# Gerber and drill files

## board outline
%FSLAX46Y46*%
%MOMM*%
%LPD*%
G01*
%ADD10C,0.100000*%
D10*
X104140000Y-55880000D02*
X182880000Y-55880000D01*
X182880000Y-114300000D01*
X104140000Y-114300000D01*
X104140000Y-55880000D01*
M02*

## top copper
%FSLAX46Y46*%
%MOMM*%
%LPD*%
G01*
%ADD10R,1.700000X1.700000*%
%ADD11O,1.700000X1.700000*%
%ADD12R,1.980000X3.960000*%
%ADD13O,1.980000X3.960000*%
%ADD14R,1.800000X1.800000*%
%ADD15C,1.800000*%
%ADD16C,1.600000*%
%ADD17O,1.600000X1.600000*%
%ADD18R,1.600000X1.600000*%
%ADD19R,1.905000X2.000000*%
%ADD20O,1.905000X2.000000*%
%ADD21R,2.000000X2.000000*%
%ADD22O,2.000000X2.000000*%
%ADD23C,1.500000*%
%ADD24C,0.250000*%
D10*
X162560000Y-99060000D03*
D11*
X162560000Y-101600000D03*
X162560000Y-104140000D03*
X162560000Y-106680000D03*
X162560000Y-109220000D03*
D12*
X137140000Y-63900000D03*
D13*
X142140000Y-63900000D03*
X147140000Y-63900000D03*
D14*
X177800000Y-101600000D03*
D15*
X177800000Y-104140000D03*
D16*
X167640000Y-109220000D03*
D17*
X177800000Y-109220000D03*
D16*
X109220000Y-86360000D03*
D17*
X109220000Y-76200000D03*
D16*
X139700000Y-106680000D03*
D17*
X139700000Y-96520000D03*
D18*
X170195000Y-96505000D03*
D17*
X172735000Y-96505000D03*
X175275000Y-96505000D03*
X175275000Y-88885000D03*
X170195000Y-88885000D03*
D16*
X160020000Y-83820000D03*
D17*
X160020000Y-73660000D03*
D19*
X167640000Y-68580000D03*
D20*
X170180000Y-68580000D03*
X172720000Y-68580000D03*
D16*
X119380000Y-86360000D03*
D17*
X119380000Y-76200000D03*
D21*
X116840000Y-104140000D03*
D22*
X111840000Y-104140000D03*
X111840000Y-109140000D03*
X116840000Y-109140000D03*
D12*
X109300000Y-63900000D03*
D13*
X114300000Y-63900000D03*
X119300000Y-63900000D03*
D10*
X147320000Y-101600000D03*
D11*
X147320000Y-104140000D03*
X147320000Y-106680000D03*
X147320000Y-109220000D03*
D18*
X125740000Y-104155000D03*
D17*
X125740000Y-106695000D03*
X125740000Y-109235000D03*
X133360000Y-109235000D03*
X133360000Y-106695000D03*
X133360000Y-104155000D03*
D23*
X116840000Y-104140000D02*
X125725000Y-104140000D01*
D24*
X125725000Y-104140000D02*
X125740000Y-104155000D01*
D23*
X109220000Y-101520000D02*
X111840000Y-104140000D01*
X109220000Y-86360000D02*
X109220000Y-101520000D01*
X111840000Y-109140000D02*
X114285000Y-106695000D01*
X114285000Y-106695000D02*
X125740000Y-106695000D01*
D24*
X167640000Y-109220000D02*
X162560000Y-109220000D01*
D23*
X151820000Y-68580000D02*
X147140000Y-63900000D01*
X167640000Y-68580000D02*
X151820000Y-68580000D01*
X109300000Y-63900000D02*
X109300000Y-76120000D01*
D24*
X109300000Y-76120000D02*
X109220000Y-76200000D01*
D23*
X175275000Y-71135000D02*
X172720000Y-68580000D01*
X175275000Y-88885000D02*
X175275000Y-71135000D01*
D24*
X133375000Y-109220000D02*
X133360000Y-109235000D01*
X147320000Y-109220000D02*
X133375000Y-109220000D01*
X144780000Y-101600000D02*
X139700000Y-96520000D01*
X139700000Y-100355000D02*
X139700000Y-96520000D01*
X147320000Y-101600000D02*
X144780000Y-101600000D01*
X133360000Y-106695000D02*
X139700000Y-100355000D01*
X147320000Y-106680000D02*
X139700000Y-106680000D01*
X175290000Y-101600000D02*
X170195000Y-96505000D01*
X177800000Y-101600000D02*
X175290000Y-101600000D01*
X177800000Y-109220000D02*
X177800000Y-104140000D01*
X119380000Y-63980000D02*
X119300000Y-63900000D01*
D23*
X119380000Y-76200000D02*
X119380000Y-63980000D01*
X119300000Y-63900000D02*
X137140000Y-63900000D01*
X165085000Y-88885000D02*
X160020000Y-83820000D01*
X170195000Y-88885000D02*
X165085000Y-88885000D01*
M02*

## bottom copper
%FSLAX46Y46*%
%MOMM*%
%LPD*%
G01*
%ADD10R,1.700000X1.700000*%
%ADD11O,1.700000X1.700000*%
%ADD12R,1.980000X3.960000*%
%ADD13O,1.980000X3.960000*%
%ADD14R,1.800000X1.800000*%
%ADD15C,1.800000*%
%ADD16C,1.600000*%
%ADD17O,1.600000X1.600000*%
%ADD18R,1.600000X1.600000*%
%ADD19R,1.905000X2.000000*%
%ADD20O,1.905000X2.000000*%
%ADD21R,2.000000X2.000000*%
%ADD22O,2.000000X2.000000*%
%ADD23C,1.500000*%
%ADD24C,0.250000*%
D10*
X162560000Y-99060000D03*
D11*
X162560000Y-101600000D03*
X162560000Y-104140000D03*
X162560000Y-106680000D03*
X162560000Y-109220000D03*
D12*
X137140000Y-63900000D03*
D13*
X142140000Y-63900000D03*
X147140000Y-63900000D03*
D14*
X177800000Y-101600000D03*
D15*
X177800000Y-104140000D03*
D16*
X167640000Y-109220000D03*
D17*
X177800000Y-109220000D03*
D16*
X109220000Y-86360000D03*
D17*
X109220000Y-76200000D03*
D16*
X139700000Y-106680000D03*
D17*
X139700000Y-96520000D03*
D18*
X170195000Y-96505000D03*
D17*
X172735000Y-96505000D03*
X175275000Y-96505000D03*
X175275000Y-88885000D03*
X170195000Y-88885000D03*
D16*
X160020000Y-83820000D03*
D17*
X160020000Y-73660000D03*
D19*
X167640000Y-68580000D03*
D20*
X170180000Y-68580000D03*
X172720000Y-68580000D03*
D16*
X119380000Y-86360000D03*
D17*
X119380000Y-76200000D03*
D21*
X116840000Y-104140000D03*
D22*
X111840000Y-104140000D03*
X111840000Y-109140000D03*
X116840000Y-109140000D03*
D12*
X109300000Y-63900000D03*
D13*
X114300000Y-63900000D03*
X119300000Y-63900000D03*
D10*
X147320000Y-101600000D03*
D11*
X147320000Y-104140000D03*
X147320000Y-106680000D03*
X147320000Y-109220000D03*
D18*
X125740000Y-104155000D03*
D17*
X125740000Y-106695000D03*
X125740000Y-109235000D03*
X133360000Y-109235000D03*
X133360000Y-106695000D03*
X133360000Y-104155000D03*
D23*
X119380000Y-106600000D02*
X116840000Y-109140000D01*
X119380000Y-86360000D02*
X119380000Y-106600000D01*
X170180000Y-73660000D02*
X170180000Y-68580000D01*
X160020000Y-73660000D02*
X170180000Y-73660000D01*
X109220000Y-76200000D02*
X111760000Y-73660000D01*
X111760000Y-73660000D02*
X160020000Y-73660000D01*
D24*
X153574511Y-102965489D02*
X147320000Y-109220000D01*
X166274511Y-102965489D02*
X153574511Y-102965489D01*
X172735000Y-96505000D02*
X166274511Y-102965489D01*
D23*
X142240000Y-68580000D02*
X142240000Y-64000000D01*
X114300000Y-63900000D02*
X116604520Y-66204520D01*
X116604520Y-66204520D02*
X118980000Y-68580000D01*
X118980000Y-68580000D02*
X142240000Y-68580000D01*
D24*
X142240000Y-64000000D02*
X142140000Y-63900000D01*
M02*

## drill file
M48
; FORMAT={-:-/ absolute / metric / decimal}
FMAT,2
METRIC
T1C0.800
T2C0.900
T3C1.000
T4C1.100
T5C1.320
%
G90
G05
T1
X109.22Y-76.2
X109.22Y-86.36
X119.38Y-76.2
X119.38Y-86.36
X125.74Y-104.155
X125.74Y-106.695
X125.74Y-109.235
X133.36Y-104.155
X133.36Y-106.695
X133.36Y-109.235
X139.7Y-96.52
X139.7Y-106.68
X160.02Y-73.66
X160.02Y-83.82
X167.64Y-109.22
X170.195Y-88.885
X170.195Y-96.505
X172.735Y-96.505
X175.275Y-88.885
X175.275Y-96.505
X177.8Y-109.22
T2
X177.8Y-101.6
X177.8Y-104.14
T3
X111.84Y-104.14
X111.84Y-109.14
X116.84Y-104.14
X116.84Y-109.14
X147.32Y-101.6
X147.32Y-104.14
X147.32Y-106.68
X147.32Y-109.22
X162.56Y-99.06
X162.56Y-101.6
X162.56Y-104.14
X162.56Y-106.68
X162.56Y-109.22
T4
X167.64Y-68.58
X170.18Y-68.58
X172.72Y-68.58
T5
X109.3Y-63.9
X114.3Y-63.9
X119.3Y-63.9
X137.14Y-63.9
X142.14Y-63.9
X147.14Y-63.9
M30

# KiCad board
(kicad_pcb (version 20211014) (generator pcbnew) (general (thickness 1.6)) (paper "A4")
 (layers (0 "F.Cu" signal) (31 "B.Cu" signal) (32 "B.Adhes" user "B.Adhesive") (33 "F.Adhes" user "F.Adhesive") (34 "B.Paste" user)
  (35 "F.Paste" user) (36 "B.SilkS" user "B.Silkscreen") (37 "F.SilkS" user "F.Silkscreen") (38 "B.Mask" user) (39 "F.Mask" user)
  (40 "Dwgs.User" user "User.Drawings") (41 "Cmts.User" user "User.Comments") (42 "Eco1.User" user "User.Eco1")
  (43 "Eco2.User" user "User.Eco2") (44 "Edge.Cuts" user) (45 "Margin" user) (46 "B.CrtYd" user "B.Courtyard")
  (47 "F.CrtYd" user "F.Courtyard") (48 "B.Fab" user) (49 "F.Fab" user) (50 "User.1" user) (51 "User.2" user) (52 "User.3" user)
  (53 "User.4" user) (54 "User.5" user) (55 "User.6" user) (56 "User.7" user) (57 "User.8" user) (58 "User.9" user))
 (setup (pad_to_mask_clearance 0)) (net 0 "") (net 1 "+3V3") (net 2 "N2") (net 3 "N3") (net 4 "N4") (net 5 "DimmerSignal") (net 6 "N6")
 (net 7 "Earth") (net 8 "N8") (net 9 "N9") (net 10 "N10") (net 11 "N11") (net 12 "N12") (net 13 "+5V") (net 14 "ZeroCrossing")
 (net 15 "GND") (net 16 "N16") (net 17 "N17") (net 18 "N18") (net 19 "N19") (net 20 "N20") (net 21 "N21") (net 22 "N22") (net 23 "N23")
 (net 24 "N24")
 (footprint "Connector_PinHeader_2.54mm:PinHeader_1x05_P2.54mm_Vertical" (layer "F.Cu") (at 162.56 99.06)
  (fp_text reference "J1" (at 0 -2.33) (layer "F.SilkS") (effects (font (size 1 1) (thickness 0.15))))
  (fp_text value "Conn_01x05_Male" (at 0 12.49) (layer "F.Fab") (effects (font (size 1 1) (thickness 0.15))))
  (pad "1" thru_hole rect (at 0 0) (size 1.7 1.7) (drill 1) (layers *.Cu *.Mask) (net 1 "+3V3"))
  (pad "2" thru_hole oval (at 0 2.54) (size 1.7 1.7) (drill 1) (layers *.Cu *.Mask) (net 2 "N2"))
  (pad "3" thru_hole oval (at 0 5.08) (size 1.7 1.7) (drill 1) (layers *.Cu *.Mask) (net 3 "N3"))
  (pad "4" thru_hole oval (at 0 7.62) (size 1.7 1.7) (drill 1) (layers *.Cu *.Mask) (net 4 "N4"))
  (pad "5" thru_hole oval (at 0 10.16) (size 1.7 1.7) (drill 1) (layers *.Cu *.Mask) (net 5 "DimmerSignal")))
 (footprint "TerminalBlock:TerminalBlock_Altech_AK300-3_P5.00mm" (layer "F.Cu") (at 137.14 63.9)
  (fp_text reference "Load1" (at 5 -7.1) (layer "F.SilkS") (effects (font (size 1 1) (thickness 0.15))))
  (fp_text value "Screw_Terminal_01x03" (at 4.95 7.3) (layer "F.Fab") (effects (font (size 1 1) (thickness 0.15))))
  (pad "1" thru_hole rect (at 0 0) (size 1.98 3.96) (drill 1.32) (layers *.Cu *.Mask) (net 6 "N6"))
  (pad "2" thru_hole oval (at 5 0) (size 1.98 3.96) (drill 1.32) (layers *.Cu *.Mask) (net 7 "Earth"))
  (pad "3" thru_hole oval (at 10 0) (size 1.98 3.96) (drill 1.32) (layers *.Cu *.Mask) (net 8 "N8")))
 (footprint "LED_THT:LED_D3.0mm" (layer "F.Cu") (at 177.8 101.6 -90)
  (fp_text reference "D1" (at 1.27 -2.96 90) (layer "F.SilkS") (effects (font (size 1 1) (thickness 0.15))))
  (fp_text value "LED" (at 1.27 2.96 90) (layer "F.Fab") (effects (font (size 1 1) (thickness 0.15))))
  (pad "1" thru_hole rect (at 0 0 270) (size 1.8 1.8) (drill 0.9) (layers *.Cu *.Mask) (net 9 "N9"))
  (pad "2" thru_hole circle (at 2.54 0 270) (size 1.8 1.8) (drill 0.9) (layers *.Cu *.Mask) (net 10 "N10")))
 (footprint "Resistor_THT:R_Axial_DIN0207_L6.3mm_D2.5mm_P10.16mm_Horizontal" (layer "F.Cu") (at 167.64 109.22)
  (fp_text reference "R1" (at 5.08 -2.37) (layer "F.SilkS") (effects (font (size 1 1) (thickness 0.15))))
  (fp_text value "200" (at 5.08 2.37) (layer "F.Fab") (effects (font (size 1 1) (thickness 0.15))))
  (pad "1" thru_hole circle (at 0 0) (size 1.6 1.6) (drill 0.8) (layers *.Cu *.Mask) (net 5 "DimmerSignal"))
  (pad "2" thru_hole oval (at 10.16 0) (size 1.6 1.6) (drill 0.8) (layers *.Cu *.Mask) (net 10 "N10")))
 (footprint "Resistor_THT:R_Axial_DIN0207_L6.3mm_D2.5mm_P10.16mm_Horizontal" (layer "F.Cu") (at 109.22 86.36 90)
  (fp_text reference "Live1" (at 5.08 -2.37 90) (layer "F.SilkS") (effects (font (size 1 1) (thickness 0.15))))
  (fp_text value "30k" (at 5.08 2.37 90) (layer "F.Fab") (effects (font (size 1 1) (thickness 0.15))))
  (pad "1" thru_hole circle (at 0 0 90) (size 1.6 1.6) (drill 0.8) (layers *.Cu *.Mask) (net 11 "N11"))
  (pad "2" thru_hole oval (at 10.16 0 90) (size 1.6 1.6) (drill 0.8) (layers *.Cu *.Mask) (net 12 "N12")))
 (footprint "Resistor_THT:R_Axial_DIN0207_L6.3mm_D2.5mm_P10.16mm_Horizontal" (layer "F.Cu") (at 139.7 106.68 90)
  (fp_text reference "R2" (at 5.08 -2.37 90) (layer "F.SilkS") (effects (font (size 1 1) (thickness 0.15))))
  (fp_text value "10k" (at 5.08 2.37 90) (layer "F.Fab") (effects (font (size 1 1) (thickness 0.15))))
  (pad "1" thru_hole circle (at 0 0 90) (size 1.6 1.6) (drill 0.8) (layers *.Cu *.Mask) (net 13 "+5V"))
  (pad "2" thru_hole oval (at 10.16 0 90) (size 1.6 1.6) (drill 0.8) (layers *.Cu *.Mask) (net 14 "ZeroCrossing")))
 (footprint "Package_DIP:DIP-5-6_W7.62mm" (layer "F.Cu") (at 170.195 96.505 90)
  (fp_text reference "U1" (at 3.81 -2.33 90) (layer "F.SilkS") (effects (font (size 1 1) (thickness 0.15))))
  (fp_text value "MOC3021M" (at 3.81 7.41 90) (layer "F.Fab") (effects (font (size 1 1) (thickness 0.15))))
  (pad "1" thru_hole rect (at 0 0 90) (size 1.6 1.6) (drill 0.8) (layers *.Cu *.Mask) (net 9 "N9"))
  (pad "2" thru_hole oval (at 0 2.54 90) (size 1.6 1.6) (drill 0.8) (layers *.Cu *.Mask) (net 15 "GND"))
  (pad "3" thru_hole oval (at 0 5.08 90) (size 1.6 1.6) (drill 0.8) (layers *.Cu *.Mask) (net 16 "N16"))
  (pad "4" thru_hole oval (at 7.62 5.08 90) (size 1.6 1.6) (drill 0.8) (layers *.Cu *.Mask) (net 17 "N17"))
  (pad "6" thru_hole oval (at 7.62 0 90) (size 1.6 1.6) (drill 0.8) (layers *.Cu *.Mask) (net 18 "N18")))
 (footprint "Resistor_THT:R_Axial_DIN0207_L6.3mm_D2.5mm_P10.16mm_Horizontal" (layer "F.Cu") (at 160.02 83.82 90)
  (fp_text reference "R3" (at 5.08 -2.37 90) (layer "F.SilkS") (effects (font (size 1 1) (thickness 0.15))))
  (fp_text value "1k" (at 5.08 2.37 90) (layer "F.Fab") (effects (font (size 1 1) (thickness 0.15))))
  (pad "1" thru_hole circle (at 0 0 90) (size 1.6 1.6) (drill 0.8) (layers *.Cu *.Mask) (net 18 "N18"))
  (pad "2" thru_hole oval (at 10.16 0 90) (size 1.6 1.6) (drill 0.8) (layers *.Cu *.Mask) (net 12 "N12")))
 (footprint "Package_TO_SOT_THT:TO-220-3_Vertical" (layer "F.Cu") (at 167.64 68.58)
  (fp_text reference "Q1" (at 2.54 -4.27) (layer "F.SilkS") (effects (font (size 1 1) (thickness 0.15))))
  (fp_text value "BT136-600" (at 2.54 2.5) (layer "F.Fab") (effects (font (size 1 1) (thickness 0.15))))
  (pad "1" thru_hole rect (at 0 0) (size 1.905 2) (drill 1.1) (layers *.Cu *.Mask) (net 8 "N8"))
  (pad "2" thru_hole oval (at 2.54 0) (size 1.905 2) (drill 1.1) (layers *.Cu *.Mask) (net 12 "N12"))
  (pad "3" thru_hole oval (at 5.08 0) (size 1.905 2) (drill 1.1) (layers *.Cu *.Mask) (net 17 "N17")))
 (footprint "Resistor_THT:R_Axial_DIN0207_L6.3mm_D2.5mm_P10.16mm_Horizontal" (layer "F.Cu") (at 119.38 86.36 90)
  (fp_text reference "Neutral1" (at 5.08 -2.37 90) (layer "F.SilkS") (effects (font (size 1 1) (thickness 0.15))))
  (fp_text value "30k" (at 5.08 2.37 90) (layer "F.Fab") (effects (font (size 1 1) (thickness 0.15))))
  (pad "1" thru_hole circle (at 0 0 90) (size 1.6 1.6) (drill 0.8) (layers *.Cu *.Mask) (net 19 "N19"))
  (pad "2" thru_hole oval (at 10.16 0 90) (size 1.6 1.6) (drill 0.8) (layers *.Cu *.Mask) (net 6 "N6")))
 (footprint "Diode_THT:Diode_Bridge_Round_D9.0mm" (layer "F.Cu") (at 116.84 104.14 -90)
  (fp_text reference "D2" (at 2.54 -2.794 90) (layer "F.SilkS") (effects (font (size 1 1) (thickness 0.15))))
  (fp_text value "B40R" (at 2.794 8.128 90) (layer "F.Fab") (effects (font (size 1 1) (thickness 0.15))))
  (pad "1" thru_hole rect (at 0 0 270) (size 2 2) (drill 1) (layers *.Cu *.Mask) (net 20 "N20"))
  (pad "2" thru_hole oval (at 0 5 270) (size 2 2) (drill 1) (layers *.Cu *.Mask) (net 11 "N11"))
  (pad "3" thru_hole oval (at 5 5 270) (size 2 2) (drill 1) (layers *.Cu *.Mask) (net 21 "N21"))
  (pad "4" thru_hole oval (at 5 0 270) (size 2 2) (drill 1) (layers *.Cu *.Mask) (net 19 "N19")))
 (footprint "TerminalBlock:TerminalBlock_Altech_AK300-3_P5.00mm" (layer "F.Cu") (at 109.3 63.9)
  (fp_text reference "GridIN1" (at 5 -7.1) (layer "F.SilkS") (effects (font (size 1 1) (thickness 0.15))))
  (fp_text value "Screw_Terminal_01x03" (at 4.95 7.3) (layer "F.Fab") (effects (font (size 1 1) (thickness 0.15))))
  (pad "1" thru_hole rect (at 0 0) (size 1.98 3.96) (drill 1.32) (layers *.Cu *.Mask) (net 12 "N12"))
  (pad "2" thru_hole oval (at 5 0) (size 1.98 3.96) (drill 1.32) (layers *.Cu *.Mask) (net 7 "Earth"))
  (pad "3" thru_hole oval (at 10 0) (size 1.98 3.96) (drill 1.32) (layers *.Cu *.Mask) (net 6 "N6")))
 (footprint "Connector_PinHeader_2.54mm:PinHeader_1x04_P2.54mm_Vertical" (layer "F.Cu") (at 147.32 101.6)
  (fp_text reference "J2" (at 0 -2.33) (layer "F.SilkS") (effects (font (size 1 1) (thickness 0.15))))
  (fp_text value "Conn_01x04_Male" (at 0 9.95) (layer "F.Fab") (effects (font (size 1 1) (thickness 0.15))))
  (pad "1" thru_hole rect (at 0 0) (size 1.7 1.7) (drill 1) (layers *.Cu *.Mask) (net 14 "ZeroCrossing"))
  (pad "2" thru_hole oval (at 0 2.54) (size 1.7 1.7) (drill 1) (layers *.Cu *.Mask) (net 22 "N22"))
  (pad "3" thru_hole oval (at 0 5.08) (size 1.7 1.7) (drill 1) (layers *.Cu *.Mask) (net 13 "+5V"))
  (pad "4" thru_hole oval (at 0 7.62) (size 1.7 1.7) (drill 1) (layers *.Cu *.Mask) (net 15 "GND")))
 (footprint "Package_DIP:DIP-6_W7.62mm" (layer "F.Cu") (at 125.74 104.155)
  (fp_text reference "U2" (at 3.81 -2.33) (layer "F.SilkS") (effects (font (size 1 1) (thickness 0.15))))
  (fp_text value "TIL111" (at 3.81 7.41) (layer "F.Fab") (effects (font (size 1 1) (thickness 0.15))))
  (pad "1" thru_hole rect (at 0 0) (size 1.6 1.6) (drill 0.8) (layers *.Cu *.Mask) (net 20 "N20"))
  (pad "2" thru_hole oval (at 0 2.54) (size 1.6 1.6) (drill 0.8) (layers *.Cu *.Mask) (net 21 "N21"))
  (pad "3" thru_hole oval (at 0 5.08) (size 1.6 1.6) (drill 0.8) (layers *.Cu *.Mask) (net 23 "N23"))
  (pad "4" thru_hole oval (at 7.62 5.08) (size 1.6 1.6) (drill 0.8) (layers *.Cu *.Mask) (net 15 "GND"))
  (pad "5" thru_hole oval (at 7.62 2.54) (size 1.6 1.6) (drill 0.8) (layers *.Cu *.Mask) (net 14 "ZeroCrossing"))
  (pad "6" thru_hole oval (at 7.62 0) (size 1.6 1.6) (drill 0.8) (layers *.Cu *.Mask) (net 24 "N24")))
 (gr_rect (start 104.14 55.88) (end 182.88 114.3) (layer "Edge.Cuts") (width 0.1) (fill none))
 (segment (start 116.84 104.14) (end 125.725 104.14) (width 1.5) (layer "F.Cu") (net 20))
 (segment (start 125.725 104.14) (end 125.74 104.155) (width 0.25) (layer "F.Cu") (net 20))
 (segment (start 109.22 101.52) (end 111.84 104.14) (width 1.5) (layer "F.Cu") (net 11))
 (segment (start 109.22 86.36) (end 109.22 101.52) (width 1.5) (layer "F.Cu") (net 11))
 (segment (start 111.84 109.14) (end 114.285 106.695) (width 1.5) (layer "F.Cu") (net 21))
 (segment (start 114.285 106.695) (end 125.74 106.695) (width 1.5) (layer "F.Cu") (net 21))
 (segment (start 119.38 106.6) (end 116.84 109.14) (width 1.5) (layer "B.Cu") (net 19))
 (segment (start 119.38 86.36) (end 119.38 106.6) (width 1.5) (layer "B.Cu") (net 19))
 (segment (start 167.64 109.22) (end 162.56 109.22) (width 0.25) (layer "F.Cu") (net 5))
 (segment (start 151.82 68.58) (end 147.14 63.9) (width 1.5) (layer "F.Cu") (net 8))
 (segment (start 167.64 68.58) (end 151.82 68.58) (width 1.5) (layer "F.Cu") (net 8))
 (segment (start 109.3 63.9) (end 109.3 76.12) (width 1.5) (layer "F.Cu") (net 12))
 (segment (start 109.3 76.12) (end 109.22 76.2) (width 0.25) (layer "F.Cu") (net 12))
 (segment (start 170.18 73.66) (end 170.18 68.58) (width 1.5) (layer "B.Cu") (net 12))
 (segment (start 160.02 73.66) (end 170.18 73.66) (width 1.5) (layer "B.Cu") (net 12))
 (segment (start 109.22 76.2) (end 111.76 73.66) (width 1.5) (layer "B.Cu") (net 12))
 (segment (start 111.76 73.66) (end 160.02 73.66) (width 1.5) (layer "B.Cu") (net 12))
 (segment (start 175.275 71.135) (end 172.72 68.58) (width 1.5) (layer "F.Cu") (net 17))
 (segment (start 175.275 88.885) (end 175.275 71.135) (width 1.5) (layer "F.Cu") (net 17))
 (segment (start 133.375 109.22) (end 133.36 109.235) (width 0.25) (layer "F.Cu") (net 15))
 (segment (start 147.32 109.22) (end 133.375 109.22) (width 0.25) (layer "F.Cu") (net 15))
 (segment (start 153.574511 102.965489) (end 147.32 109.22) (width 0.25) (layer "B.Cu") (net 15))
 (segment (start 166.274511 102.965489) (end 153.574511 102.965489) (width 0.25) (layer "B.Cu") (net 15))
 (segment (start 172.735 96.505) (end 166.274511 102.965489) (width 0.25) (layer "B.Cu") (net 15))
 (segment (start 144.78 101.6) (end 139.7 96.52) (width 0.25) (layer "F.Cu") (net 14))
 (segment (start 139.7 100.355) (end 139.7 96.52) (width 0.25) (layer "F.Cu") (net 14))
 (segment (start 147.32 101.6) (end 144.78 101.6) (width 0.25) (layer "F.Cu") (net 14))
 (segment (start 133.36 106.695) (end 139.7 100.355) (width 0.25) (layer "F.Cu") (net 14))
 (segment (start 147.32 106.68) (end 139.7 106.68) (width 0.25) (layer "F.Cu") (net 13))
 (segment (start 175.29 101.6) (end 170.195 96.505) (width 0.25) (layer "F.Cu") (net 9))
 (segment (start 177.8 101.6) (end 175.29 101.6) (width 0.25) (layer "F.Cu") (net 9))
 (segment (start 177.8 109.22) (end 177.8 104.14) (width 0.25) (layer "F.Cu") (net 10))
 (segment (start 142.24 68.58) (end 142.24 64) (width 1.5) (layer "B.Cu") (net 7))
 (segment (start 114.3 63.9) (end 116.60452 66.20452) (width 1.5) (layer "B.Cu") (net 7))
 (segment (start 116.60452 66.20452) (end 118.98 68.58) (width 1.5) (layer "B.Cu") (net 7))
 (segment (start 118.98 68.58) (end 142.24 68.58) (width 1.5) (layer "B.Cu") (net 7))
 (segment (start 142.24 64) (end 142.14 63.9) (width 0.25) (layer "B.Cu") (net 7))
 (segment (start 119.38 63.98) (end 119.3 63.9) (width 0.25) (layer "F.Cu") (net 6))
 (segment (start 119.38 76.2) (end 119.38 63.98) (width 1.5) (layer "F.Cu") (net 6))
 (segment (start 119.3 63.9) (end 137.14 63.9) (width 1.5) (layer "F.Cu") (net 6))
 (segment (start 165.085 88.885) (end 160.02 83.82) (width 1.5) (layer "F.Cu") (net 18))
 (segment (start 170.195 88.885) (end 165.085 88.885) (width 1.5) (layer "F.Cu") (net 18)))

